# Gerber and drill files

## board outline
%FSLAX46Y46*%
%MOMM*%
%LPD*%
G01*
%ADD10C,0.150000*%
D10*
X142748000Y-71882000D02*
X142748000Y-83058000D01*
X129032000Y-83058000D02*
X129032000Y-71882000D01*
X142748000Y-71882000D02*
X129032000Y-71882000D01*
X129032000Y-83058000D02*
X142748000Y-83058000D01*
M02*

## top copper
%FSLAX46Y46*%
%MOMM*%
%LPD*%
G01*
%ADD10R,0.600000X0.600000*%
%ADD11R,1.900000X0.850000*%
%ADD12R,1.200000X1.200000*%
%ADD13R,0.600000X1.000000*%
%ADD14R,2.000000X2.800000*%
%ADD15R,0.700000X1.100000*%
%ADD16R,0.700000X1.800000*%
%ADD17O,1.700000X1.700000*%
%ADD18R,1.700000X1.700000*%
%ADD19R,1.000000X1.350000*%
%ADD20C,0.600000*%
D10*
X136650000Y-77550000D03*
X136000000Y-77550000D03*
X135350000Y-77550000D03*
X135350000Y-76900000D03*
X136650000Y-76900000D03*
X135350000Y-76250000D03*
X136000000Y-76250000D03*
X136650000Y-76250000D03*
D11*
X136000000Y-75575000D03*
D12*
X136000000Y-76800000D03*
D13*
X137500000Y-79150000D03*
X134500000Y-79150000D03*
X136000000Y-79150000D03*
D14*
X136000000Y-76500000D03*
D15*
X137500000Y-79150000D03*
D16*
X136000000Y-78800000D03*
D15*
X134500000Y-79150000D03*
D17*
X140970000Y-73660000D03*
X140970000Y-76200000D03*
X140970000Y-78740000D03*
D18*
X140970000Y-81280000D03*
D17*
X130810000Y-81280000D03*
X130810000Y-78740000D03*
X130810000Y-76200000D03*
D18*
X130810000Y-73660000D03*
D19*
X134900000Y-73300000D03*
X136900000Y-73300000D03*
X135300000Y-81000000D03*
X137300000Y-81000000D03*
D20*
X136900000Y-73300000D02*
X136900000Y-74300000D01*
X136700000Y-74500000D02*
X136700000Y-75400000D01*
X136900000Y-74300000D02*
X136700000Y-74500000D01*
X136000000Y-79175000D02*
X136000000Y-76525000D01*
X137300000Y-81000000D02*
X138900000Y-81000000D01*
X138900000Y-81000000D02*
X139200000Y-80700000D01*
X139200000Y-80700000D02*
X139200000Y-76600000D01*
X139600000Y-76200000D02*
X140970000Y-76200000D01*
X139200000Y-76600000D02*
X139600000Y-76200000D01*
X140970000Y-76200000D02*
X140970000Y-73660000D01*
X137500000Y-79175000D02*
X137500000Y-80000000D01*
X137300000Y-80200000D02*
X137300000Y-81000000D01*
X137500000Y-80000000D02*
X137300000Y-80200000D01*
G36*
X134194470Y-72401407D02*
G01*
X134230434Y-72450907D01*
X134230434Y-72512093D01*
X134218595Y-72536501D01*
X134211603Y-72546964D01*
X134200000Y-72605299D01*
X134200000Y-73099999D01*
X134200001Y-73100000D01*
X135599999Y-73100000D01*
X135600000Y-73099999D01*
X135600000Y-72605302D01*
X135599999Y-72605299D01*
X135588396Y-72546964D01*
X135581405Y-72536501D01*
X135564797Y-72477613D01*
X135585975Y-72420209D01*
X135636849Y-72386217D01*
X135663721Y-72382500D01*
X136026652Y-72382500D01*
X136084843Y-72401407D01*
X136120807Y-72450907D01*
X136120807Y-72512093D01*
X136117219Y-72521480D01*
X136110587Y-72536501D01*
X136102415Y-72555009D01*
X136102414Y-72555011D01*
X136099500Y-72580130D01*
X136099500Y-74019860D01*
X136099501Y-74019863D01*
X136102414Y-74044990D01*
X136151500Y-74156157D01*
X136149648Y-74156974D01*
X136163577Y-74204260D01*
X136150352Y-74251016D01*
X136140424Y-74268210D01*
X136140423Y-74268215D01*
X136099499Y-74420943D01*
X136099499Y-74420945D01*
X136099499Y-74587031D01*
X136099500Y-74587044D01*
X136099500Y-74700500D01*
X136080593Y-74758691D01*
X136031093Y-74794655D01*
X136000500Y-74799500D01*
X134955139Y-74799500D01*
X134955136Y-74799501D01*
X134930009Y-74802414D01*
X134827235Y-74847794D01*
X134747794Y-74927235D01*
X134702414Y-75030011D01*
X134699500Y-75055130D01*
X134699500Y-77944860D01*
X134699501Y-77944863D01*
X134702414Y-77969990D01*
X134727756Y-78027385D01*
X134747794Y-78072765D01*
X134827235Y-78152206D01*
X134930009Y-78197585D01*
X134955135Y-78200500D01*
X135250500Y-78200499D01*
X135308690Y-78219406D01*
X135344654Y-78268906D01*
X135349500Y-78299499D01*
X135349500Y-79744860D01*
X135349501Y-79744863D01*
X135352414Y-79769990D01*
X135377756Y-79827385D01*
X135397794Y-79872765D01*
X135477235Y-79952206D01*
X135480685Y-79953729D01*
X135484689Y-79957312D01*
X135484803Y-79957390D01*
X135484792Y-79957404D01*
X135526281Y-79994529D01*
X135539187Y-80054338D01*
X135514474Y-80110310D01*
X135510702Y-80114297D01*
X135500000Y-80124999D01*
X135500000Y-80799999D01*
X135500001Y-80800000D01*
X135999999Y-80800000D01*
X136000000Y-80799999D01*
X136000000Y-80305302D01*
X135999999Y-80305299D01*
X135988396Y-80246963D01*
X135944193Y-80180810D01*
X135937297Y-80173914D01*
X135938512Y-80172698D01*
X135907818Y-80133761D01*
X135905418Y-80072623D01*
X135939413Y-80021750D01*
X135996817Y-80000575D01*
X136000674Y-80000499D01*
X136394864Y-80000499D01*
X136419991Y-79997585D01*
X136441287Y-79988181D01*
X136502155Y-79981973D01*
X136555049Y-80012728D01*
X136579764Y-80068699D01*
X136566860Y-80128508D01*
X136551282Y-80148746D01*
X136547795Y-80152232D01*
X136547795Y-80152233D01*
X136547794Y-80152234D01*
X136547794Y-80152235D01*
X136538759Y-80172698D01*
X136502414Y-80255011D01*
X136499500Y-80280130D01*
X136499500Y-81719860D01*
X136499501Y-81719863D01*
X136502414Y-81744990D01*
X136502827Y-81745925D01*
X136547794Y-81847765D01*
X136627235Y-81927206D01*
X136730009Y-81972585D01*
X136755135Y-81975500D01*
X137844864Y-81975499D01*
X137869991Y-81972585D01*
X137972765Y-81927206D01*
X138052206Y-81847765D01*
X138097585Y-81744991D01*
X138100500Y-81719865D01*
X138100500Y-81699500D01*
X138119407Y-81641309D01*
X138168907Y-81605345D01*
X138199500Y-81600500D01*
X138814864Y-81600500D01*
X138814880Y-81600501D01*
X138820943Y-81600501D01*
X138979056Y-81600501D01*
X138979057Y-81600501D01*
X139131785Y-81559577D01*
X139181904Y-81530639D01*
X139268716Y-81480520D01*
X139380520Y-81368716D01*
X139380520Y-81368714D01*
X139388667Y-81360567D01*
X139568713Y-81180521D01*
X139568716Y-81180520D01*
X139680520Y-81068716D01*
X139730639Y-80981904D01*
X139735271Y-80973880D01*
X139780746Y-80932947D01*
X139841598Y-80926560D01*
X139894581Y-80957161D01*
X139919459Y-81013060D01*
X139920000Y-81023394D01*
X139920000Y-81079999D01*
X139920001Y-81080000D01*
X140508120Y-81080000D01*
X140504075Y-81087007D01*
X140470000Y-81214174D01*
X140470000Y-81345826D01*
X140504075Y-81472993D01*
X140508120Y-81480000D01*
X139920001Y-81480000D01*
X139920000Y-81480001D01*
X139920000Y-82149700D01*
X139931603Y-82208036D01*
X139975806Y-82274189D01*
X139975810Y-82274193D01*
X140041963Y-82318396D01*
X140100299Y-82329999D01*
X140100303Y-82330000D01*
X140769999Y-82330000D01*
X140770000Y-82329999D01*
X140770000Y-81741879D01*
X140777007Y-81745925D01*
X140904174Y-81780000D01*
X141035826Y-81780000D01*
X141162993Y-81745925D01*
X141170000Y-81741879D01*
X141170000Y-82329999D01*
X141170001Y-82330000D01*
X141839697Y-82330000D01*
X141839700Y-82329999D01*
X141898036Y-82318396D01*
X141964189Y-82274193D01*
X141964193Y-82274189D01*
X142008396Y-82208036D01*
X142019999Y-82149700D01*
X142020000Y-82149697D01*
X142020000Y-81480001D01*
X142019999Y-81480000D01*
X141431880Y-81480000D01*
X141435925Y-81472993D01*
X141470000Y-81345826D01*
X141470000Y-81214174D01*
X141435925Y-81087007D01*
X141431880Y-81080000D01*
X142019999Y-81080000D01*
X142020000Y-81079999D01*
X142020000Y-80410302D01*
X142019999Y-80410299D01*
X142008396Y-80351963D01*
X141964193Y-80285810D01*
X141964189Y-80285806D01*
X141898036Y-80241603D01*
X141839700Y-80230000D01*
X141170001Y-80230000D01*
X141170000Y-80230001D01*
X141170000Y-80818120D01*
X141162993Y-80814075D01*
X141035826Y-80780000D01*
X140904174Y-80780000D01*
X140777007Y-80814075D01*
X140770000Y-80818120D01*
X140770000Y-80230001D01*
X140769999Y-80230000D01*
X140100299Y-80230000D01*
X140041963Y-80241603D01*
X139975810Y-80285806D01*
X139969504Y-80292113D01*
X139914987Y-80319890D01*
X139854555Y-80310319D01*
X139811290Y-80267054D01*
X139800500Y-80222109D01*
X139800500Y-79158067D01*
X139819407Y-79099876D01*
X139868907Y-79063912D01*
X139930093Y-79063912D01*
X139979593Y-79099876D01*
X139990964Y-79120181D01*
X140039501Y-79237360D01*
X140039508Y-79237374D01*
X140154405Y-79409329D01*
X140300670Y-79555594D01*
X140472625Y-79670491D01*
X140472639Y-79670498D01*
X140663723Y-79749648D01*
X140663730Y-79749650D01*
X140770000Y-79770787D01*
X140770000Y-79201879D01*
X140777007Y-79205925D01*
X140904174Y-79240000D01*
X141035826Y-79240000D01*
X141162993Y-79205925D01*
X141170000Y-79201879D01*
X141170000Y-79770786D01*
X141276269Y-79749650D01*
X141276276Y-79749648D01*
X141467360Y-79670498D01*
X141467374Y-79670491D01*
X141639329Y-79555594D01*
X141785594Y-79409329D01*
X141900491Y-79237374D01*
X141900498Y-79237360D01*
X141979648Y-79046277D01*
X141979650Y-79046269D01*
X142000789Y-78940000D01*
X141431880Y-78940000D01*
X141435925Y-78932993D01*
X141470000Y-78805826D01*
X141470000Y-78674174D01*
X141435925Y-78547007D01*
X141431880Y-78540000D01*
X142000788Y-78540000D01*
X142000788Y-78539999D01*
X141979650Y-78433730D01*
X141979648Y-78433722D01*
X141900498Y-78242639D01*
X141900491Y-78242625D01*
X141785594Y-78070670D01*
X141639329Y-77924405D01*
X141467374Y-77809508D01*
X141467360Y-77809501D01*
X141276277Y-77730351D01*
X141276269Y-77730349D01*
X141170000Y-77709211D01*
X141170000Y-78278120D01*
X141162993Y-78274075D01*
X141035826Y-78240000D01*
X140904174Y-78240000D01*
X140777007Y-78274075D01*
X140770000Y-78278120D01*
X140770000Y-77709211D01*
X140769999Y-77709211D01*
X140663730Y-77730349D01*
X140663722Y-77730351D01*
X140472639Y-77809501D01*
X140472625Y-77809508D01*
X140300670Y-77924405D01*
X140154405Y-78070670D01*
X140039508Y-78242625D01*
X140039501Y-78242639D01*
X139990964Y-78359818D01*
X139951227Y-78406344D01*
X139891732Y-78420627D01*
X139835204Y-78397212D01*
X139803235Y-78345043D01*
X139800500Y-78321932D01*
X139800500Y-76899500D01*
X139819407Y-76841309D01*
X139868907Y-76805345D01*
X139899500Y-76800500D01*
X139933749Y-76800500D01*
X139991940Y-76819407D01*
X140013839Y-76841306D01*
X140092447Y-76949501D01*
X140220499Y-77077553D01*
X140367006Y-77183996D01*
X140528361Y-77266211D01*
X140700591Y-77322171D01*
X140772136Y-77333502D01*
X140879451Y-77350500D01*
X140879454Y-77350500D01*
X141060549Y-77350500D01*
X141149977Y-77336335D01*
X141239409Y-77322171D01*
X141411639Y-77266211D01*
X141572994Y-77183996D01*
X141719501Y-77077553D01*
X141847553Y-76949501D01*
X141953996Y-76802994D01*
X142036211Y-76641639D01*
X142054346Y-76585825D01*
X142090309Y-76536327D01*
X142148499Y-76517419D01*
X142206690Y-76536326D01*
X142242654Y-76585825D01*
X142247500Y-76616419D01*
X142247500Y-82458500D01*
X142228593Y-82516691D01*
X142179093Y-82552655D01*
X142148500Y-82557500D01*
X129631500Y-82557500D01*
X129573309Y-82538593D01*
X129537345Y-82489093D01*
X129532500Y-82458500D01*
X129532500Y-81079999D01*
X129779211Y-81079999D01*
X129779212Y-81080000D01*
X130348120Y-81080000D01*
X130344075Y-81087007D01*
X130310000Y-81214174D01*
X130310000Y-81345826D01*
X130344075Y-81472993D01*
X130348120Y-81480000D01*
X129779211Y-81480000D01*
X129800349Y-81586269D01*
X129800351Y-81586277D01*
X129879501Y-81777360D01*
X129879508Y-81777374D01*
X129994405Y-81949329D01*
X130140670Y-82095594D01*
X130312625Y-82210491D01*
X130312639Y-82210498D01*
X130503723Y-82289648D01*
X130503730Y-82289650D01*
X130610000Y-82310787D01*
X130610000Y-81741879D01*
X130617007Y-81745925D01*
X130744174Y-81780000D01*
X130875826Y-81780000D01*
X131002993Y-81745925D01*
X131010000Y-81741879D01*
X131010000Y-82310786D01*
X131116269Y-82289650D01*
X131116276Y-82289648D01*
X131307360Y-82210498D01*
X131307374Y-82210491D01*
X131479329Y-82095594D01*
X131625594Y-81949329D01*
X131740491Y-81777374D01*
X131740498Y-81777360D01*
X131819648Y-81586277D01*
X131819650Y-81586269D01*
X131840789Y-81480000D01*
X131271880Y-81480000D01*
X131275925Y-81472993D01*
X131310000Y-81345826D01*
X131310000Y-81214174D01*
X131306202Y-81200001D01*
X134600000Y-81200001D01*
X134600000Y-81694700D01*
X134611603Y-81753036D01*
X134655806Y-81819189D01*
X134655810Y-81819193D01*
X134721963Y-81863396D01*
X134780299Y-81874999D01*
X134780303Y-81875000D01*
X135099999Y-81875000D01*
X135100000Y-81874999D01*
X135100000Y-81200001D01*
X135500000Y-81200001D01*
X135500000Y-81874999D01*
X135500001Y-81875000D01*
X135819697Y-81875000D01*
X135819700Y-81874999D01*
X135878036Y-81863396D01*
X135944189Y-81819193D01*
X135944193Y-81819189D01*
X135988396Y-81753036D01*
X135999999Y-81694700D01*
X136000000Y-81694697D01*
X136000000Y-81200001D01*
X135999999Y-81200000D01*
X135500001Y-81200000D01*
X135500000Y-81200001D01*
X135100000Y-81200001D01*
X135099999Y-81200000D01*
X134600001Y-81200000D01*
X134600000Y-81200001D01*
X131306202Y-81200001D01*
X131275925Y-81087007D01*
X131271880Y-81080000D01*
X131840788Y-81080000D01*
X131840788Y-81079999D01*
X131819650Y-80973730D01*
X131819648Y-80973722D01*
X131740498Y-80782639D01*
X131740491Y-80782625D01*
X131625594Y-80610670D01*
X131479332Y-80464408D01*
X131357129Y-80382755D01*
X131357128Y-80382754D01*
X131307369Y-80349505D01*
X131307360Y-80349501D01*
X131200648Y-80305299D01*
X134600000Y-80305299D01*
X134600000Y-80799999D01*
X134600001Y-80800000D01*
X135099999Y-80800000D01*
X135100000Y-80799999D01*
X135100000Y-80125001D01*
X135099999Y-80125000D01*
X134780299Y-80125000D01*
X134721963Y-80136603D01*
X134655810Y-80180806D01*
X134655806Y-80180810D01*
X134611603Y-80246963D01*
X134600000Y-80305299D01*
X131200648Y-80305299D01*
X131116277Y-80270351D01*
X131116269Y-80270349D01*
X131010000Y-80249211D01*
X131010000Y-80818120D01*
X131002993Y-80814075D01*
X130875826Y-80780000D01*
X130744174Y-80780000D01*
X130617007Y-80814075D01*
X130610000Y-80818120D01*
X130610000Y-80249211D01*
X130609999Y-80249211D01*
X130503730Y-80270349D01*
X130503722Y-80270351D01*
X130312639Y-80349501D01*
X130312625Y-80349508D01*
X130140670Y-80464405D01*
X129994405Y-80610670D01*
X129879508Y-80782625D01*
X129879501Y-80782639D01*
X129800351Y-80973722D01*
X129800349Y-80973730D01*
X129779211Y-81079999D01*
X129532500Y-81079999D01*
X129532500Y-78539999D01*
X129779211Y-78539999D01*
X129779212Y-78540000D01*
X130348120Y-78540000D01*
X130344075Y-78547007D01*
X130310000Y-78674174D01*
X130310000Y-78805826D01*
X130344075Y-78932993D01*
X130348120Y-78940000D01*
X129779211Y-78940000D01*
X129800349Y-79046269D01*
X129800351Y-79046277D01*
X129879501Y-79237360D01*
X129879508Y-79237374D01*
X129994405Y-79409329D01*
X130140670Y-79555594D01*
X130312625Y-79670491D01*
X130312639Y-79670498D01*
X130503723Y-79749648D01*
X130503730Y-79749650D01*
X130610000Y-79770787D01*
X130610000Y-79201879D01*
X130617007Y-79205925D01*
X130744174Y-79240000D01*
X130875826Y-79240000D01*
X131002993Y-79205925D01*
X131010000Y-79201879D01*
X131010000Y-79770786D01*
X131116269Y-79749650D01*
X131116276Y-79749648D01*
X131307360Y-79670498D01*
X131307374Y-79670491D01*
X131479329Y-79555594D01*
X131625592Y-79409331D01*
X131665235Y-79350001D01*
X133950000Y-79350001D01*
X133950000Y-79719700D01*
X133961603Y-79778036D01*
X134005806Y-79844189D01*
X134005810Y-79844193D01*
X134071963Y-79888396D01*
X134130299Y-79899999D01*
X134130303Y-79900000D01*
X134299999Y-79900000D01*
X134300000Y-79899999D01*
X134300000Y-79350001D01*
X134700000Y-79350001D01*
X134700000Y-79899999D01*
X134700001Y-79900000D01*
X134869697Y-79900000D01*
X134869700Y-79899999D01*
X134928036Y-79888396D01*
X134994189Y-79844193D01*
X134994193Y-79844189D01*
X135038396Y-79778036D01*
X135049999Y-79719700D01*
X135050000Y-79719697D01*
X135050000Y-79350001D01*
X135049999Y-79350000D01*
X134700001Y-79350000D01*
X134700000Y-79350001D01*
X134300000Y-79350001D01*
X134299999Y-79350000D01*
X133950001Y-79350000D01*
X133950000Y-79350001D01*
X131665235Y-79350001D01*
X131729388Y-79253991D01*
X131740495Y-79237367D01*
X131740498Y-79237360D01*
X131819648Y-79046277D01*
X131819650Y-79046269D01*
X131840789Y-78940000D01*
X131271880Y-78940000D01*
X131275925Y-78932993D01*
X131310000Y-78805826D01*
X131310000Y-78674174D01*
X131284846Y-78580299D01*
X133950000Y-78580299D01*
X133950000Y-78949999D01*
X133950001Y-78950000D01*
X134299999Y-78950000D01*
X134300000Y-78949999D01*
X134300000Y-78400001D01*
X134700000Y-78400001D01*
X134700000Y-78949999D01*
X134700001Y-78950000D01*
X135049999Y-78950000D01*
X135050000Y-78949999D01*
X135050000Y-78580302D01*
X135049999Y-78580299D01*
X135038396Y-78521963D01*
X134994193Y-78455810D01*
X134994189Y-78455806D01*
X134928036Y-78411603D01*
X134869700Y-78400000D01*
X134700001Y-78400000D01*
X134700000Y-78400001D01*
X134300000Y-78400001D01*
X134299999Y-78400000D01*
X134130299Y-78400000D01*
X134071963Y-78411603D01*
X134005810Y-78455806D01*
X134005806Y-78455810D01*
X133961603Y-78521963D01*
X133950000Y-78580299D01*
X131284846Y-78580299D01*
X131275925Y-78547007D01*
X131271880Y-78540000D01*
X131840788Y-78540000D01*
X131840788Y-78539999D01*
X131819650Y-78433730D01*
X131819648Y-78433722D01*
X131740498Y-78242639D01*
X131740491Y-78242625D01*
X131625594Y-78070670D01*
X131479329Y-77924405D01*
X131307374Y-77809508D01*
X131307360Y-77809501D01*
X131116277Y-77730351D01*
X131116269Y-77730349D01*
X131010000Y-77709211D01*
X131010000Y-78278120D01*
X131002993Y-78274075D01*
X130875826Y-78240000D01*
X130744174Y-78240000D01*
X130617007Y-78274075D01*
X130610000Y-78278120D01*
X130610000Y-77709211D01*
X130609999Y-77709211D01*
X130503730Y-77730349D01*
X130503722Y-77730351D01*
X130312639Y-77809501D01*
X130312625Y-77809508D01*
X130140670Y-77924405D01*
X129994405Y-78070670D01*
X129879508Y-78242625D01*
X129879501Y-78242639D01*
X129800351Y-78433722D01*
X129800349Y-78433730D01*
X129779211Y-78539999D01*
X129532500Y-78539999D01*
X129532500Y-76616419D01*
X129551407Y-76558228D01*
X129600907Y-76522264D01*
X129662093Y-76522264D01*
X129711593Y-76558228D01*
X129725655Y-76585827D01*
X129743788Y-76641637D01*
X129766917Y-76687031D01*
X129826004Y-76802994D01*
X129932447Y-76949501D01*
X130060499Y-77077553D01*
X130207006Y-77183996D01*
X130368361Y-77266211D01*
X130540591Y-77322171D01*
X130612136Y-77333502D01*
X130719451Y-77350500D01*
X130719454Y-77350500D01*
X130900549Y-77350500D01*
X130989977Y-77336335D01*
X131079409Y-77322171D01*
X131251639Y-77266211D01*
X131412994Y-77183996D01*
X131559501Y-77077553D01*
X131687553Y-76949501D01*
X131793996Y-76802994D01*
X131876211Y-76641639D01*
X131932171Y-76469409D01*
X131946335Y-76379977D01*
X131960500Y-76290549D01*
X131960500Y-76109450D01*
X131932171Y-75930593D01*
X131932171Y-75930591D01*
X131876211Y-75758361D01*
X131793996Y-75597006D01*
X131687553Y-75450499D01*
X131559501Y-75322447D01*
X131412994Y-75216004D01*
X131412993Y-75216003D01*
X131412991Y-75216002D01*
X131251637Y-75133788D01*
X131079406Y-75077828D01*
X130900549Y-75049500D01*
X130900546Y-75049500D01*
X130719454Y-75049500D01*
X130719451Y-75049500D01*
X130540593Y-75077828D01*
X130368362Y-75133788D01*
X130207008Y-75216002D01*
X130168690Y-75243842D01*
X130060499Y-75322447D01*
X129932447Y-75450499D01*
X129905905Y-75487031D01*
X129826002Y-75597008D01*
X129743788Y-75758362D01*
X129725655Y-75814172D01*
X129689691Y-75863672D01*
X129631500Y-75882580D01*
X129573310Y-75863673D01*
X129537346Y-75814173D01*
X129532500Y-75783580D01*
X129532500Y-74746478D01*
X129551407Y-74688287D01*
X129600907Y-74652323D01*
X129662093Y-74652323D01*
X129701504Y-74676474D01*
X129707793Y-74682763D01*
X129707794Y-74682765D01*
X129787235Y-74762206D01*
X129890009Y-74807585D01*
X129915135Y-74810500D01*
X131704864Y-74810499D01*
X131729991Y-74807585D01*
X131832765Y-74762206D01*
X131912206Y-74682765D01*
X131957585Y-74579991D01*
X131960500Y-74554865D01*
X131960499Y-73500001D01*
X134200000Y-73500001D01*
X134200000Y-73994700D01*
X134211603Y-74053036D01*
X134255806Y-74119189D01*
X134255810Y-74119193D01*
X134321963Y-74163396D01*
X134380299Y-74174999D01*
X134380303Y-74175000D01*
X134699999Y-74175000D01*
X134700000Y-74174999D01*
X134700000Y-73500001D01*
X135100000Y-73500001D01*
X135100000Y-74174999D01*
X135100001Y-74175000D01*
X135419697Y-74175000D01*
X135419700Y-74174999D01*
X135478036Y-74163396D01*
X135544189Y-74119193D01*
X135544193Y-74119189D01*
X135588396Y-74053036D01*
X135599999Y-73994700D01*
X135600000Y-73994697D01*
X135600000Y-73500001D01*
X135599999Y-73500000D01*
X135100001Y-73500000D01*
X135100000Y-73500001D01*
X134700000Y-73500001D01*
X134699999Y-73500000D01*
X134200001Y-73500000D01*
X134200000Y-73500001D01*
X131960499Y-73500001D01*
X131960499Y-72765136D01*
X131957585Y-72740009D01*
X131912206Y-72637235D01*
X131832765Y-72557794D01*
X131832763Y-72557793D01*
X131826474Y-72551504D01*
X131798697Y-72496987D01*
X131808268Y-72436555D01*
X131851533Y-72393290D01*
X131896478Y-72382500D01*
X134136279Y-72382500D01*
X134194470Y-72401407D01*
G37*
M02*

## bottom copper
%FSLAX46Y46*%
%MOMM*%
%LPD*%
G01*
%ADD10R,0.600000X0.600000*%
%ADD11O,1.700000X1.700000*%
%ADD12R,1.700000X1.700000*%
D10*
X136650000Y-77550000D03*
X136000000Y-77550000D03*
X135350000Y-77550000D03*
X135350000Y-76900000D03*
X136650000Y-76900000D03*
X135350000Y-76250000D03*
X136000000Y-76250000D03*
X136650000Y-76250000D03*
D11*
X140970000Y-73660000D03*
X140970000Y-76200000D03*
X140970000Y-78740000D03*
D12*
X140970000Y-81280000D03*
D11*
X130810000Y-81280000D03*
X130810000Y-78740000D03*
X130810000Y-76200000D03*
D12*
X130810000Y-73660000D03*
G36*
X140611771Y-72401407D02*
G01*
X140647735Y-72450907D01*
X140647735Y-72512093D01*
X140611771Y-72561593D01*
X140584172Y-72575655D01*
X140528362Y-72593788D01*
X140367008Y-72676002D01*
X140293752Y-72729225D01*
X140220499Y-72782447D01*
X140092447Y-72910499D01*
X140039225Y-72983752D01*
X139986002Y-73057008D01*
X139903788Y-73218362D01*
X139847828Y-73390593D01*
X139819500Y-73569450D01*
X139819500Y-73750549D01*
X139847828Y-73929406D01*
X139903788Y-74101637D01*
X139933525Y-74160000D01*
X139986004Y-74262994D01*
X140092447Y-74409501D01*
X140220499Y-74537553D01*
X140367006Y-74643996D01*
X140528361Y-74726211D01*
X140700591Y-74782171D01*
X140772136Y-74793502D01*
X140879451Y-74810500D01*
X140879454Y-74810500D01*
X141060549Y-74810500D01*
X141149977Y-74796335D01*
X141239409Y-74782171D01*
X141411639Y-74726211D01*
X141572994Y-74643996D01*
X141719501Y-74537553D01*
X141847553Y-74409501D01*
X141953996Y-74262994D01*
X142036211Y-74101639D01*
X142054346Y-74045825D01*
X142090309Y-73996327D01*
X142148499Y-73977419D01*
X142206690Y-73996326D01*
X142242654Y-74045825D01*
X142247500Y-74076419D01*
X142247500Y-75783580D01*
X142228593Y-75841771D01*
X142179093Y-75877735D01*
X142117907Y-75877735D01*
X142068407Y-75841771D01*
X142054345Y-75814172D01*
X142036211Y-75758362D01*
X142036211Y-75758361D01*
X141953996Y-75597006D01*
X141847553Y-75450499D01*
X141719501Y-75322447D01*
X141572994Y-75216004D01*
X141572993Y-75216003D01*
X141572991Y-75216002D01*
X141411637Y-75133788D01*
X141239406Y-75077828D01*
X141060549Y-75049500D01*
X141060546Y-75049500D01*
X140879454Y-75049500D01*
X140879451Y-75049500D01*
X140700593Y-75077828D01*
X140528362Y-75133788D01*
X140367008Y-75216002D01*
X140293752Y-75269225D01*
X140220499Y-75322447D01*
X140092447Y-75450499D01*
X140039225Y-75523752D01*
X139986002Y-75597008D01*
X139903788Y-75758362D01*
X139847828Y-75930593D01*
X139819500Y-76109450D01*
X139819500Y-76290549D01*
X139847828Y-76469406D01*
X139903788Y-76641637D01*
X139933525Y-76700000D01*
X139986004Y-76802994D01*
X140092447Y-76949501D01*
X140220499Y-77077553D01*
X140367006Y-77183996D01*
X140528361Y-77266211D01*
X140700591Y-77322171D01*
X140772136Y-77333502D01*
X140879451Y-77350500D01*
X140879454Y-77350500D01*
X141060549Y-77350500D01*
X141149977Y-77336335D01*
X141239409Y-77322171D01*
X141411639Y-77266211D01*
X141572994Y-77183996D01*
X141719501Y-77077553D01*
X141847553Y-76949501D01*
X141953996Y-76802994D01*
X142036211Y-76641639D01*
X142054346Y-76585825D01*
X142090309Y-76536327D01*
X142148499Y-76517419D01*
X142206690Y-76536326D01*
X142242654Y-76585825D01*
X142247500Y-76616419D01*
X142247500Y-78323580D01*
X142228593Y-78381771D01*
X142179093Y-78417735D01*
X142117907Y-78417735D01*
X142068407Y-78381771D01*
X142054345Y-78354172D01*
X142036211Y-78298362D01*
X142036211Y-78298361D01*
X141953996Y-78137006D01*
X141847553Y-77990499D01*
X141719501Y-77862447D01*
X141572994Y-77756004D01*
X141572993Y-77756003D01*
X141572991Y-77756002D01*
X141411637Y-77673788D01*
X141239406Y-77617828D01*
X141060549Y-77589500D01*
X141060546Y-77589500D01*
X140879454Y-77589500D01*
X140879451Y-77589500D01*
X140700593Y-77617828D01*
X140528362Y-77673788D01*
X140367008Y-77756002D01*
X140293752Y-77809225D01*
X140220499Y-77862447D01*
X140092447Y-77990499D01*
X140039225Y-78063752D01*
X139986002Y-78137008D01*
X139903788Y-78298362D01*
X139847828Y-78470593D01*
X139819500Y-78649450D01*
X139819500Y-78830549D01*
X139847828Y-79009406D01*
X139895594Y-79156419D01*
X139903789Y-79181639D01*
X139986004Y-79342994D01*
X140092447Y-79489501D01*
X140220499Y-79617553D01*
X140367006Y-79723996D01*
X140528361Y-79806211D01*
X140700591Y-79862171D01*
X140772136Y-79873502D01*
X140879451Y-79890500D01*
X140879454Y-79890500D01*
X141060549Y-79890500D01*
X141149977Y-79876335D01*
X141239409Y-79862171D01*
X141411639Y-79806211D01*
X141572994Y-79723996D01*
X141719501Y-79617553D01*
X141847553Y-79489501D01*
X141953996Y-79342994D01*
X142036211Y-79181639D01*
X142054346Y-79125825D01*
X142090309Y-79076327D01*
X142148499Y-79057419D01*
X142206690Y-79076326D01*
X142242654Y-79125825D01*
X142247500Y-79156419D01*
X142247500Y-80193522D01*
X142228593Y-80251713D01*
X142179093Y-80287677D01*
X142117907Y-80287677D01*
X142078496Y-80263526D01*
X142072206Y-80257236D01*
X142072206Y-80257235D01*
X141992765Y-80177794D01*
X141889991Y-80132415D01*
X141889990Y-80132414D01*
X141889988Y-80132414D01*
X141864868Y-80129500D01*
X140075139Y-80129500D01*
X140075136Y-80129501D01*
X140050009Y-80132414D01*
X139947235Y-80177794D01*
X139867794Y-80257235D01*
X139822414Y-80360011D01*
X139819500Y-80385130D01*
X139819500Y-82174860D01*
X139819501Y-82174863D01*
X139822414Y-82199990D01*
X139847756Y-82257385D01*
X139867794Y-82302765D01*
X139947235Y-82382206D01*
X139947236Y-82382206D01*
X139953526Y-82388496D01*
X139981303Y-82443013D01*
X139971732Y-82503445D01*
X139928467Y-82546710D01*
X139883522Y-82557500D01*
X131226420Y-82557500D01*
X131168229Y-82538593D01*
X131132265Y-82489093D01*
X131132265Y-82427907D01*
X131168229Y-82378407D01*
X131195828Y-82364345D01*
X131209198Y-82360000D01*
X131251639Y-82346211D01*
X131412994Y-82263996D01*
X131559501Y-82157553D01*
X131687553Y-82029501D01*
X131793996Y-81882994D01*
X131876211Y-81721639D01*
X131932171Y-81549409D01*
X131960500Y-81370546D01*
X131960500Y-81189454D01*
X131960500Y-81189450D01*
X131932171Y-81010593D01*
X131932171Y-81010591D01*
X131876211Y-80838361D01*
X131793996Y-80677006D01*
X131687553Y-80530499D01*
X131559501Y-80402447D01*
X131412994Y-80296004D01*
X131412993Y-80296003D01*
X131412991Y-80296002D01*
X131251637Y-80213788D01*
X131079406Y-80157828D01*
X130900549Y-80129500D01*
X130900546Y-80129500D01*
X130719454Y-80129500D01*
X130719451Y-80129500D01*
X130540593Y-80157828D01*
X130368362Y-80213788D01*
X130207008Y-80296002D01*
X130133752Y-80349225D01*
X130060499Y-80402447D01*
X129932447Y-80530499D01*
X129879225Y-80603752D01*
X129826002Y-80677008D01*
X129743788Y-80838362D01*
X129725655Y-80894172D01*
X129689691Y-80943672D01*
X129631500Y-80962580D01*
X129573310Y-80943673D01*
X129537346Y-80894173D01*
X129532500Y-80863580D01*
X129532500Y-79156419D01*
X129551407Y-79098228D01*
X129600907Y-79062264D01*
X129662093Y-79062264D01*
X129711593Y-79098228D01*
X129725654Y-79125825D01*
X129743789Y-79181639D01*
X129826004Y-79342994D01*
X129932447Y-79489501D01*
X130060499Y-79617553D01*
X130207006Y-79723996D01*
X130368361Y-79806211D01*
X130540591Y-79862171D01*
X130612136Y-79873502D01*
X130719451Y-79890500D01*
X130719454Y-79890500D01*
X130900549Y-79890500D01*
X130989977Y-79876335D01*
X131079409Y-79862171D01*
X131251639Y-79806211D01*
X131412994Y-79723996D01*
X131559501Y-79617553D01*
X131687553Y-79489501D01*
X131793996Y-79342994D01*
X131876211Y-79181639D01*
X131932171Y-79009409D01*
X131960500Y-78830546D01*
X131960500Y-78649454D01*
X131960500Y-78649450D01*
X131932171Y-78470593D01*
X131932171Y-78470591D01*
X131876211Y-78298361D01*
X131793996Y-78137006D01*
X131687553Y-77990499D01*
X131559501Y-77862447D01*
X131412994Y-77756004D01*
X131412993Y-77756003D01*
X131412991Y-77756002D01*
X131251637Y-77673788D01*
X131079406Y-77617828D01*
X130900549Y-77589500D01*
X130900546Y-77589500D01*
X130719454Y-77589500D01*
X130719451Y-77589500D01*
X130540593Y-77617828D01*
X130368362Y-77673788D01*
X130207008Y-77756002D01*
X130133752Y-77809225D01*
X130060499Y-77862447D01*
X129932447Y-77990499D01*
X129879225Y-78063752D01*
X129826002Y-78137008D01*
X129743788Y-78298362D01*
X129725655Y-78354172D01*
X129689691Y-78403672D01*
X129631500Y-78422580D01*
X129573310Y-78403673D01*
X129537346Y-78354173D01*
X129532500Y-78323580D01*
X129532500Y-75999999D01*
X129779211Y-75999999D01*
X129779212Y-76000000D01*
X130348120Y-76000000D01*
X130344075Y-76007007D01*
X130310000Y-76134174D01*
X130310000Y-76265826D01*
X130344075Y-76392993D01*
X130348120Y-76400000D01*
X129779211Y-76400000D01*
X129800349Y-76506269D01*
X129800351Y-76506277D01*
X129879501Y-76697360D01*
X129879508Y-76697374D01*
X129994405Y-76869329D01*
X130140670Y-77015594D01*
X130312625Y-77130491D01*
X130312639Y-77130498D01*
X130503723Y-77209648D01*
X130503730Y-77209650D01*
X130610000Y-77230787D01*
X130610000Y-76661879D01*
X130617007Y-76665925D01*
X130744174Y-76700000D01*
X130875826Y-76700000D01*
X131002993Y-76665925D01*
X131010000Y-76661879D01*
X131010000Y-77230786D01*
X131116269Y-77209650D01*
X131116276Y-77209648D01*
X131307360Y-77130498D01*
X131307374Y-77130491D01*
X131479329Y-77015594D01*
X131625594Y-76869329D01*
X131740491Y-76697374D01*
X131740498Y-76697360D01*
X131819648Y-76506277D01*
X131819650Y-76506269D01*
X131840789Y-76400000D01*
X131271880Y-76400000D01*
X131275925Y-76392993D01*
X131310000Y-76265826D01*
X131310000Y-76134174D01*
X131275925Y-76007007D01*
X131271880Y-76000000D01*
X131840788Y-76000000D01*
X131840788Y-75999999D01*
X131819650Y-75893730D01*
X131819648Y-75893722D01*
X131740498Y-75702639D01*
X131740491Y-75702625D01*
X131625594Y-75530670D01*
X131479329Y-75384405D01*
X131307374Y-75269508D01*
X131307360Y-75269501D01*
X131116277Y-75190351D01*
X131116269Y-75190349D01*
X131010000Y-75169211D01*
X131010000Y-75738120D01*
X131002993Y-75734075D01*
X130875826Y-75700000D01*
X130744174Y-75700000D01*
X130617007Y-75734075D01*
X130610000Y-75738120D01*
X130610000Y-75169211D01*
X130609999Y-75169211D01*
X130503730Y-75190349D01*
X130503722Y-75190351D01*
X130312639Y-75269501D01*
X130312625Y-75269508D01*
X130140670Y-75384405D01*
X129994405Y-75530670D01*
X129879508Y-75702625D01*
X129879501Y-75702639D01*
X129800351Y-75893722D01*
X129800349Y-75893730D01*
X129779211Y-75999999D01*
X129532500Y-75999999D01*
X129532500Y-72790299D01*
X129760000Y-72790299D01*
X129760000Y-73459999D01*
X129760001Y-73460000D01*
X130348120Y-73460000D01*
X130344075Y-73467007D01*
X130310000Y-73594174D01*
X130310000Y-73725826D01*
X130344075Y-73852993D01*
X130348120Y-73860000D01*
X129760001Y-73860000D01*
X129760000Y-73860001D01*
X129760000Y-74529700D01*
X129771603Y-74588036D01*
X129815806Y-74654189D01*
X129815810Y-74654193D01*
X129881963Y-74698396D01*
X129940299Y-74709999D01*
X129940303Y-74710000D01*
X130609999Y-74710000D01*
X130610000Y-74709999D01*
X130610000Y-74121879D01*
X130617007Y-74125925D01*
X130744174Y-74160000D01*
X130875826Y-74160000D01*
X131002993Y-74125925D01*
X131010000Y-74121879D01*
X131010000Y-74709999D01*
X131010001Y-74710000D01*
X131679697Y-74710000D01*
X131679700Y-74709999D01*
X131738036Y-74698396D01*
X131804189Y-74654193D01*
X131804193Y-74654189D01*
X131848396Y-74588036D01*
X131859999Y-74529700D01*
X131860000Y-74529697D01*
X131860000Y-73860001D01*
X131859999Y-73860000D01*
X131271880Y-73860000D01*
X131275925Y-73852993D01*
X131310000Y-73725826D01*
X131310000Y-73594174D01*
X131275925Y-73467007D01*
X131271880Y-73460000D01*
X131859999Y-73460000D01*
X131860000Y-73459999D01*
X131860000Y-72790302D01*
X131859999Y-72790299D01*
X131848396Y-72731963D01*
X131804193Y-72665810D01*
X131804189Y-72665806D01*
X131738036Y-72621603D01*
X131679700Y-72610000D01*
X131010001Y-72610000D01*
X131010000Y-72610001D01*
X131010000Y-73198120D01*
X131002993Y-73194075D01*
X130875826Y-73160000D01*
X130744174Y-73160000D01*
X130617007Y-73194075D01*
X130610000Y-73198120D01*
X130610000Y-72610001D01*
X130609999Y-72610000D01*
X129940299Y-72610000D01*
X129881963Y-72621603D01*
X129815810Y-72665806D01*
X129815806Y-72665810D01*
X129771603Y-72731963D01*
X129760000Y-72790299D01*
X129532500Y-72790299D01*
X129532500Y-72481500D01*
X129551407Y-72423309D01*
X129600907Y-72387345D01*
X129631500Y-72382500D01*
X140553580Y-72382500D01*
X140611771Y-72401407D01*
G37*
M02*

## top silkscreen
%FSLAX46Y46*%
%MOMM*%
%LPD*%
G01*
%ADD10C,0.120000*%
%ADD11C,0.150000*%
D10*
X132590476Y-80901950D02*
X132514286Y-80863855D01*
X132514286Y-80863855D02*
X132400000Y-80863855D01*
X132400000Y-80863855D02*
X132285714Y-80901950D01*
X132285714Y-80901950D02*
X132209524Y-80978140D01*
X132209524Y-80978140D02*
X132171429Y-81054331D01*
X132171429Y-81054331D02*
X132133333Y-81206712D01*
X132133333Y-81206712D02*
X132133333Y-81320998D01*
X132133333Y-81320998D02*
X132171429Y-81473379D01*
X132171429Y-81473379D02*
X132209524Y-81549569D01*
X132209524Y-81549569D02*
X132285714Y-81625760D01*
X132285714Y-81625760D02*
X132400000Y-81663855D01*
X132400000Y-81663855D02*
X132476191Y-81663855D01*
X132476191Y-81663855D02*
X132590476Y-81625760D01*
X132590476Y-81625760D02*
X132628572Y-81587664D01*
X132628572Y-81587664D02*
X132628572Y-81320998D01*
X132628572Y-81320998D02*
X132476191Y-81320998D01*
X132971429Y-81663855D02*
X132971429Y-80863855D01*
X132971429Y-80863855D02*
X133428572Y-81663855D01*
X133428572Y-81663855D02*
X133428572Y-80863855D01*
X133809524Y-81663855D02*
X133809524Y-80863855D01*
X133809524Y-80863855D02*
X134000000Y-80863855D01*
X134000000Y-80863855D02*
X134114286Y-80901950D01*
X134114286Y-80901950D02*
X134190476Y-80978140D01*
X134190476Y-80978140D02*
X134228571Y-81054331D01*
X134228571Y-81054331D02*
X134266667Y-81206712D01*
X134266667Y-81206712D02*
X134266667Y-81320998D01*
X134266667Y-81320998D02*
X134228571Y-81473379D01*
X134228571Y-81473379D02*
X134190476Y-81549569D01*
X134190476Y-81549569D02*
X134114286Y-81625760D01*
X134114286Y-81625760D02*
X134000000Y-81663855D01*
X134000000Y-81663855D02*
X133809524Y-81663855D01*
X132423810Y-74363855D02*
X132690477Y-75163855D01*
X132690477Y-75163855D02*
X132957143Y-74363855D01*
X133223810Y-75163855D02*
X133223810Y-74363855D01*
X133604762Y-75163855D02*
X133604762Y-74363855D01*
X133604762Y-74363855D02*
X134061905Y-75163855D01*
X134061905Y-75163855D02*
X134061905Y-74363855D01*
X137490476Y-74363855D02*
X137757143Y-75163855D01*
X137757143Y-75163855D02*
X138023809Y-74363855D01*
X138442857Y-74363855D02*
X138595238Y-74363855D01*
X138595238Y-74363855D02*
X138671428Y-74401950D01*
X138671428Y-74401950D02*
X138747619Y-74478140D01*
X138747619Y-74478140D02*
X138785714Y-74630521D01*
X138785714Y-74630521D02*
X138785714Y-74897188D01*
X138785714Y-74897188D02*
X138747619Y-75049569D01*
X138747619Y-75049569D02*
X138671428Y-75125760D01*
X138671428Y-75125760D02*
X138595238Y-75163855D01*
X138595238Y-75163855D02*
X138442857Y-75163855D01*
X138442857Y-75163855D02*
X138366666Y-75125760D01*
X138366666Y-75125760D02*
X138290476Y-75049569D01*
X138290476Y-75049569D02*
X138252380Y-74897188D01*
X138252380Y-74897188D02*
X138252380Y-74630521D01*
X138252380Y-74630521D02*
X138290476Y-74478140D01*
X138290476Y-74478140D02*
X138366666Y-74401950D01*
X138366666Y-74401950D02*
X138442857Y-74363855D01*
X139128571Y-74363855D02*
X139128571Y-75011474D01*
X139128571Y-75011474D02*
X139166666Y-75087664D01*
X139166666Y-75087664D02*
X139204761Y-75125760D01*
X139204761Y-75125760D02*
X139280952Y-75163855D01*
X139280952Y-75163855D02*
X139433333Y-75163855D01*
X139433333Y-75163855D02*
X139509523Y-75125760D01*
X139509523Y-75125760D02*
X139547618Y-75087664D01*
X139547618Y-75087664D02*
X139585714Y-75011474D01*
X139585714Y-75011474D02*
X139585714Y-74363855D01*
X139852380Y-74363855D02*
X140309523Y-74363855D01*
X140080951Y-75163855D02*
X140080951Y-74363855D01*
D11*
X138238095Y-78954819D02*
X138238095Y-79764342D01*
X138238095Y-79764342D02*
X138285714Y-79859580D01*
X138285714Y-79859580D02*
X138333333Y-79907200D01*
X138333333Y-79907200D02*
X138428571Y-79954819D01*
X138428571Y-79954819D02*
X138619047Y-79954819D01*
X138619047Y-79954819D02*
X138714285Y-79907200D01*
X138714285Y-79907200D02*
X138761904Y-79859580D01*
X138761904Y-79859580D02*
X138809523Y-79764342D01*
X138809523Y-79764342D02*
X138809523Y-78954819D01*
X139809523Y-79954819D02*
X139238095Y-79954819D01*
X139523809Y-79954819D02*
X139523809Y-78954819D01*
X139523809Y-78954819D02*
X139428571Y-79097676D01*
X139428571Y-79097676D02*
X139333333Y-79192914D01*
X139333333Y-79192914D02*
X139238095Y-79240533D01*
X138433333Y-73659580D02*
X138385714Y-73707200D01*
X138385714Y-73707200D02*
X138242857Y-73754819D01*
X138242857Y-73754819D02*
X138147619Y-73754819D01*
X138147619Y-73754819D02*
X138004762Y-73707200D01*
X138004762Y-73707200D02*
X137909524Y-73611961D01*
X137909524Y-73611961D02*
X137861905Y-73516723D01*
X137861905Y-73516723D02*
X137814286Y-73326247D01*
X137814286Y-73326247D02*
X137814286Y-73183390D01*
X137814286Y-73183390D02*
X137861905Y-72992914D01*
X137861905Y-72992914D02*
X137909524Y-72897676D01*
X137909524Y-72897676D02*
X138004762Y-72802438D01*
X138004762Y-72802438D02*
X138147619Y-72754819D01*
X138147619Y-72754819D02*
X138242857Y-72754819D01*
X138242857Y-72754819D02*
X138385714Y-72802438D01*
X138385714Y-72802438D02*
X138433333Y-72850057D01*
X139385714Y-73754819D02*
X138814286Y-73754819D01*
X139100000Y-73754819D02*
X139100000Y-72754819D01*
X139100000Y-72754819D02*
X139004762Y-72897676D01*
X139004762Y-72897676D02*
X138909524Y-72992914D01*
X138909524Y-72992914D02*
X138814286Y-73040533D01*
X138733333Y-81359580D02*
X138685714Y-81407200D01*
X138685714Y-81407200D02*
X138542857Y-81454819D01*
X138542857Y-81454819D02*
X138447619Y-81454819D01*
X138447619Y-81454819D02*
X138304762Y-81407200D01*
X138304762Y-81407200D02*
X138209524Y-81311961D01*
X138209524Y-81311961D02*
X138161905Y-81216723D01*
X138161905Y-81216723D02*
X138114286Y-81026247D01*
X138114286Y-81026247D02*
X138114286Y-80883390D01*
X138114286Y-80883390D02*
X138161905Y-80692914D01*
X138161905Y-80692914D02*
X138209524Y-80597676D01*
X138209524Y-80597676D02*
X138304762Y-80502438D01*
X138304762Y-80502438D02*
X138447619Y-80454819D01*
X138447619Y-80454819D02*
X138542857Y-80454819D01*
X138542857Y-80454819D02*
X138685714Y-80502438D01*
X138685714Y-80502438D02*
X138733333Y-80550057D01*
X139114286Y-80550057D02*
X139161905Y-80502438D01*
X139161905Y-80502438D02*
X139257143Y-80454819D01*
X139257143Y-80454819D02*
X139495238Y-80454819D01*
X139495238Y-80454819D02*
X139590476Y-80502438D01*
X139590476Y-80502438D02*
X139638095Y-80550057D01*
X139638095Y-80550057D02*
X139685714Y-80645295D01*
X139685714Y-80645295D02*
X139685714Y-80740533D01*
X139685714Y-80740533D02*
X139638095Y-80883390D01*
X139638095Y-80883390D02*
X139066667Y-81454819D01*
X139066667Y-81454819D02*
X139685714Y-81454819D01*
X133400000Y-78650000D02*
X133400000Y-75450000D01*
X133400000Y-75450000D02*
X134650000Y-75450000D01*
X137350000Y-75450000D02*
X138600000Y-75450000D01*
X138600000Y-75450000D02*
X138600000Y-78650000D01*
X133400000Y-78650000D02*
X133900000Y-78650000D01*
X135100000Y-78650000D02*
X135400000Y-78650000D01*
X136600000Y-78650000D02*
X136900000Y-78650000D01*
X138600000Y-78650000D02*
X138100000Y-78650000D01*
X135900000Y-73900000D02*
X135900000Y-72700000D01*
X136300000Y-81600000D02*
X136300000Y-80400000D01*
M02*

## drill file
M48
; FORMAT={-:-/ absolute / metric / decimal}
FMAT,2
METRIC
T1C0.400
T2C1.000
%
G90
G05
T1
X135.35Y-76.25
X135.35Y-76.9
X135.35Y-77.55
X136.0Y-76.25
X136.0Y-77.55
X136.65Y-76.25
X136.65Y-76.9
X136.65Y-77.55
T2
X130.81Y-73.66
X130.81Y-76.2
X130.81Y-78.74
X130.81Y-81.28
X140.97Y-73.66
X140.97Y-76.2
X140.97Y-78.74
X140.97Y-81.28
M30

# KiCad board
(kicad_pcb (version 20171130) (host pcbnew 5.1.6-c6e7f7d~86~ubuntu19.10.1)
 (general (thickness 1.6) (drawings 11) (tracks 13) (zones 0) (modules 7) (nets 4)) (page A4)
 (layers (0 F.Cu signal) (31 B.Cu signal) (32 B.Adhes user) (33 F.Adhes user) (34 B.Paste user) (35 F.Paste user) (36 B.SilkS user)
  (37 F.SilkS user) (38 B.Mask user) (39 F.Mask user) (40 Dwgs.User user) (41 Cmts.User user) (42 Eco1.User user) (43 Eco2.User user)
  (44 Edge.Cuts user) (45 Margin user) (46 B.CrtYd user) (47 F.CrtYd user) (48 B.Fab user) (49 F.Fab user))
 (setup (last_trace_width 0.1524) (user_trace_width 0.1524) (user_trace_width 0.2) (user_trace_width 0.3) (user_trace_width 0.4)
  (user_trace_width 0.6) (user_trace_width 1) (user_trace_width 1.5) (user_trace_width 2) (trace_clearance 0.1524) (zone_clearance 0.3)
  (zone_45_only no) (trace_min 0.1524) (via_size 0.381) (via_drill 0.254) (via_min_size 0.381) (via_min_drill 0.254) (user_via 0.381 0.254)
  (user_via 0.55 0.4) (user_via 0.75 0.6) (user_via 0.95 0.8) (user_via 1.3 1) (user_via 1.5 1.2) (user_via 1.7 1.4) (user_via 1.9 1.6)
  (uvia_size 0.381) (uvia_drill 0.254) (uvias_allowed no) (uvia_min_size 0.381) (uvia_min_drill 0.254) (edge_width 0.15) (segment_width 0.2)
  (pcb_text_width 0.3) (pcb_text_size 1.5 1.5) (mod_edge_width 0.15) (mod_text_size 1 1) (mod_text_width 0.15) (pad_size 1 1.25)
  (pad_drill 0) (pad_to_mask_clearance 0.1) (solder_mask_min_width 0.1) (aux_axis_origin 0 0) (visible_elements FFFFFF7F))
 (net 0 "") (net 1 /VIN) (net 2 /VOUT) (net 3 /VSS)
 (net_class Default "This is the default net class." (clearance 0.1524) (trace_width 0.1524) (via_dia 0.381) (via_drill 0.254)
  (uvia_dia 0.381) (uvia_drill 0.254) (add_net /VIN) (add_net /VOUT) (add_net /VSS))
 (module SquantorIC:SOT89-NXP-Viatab (layer F.Cu) (at 136 77.4)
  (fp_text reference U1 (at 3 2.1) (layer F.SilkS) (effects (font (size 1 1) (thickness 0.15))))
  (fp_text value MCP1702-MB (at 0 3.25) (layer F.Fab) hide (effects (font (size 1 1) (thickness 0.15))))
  (fp_line (start -2.6 1.25) (end -2.6 -1.95) (layer F.SilkS) (width 0.15))
  (fp_line (start -2.6 -1.95) (end -1.35 -1.95) (layer F.SilkS) (width 0.15))
  (fp_line (start 1.35 -1.95) (end 2.6 -1.95) (layer F.SilkS) (width 0.15))
  (fp_line (start 2.6 -1.95) (end 2.6 1.25) (layer F.SilkS) (width 0.15))
  (fp_line (start -2.6 1.25) (end -2.1 1.25) (layer F.SilkS) (width 0.15))
  (fp_line (start -0.9 1.25) (end -0.6 1.25) (layer F.SilkS) (width 0.15))
  (fp_line (start 0.6 1.25) (end 0.9 1.25) (layer F.SilkS) (width 0.15))
  (fp_line (start 2.6 1.25) (end 2.1 1.25) (layer F.SilkS) (width 0.15))
  (pad 2 thru_hole rect (at 0.65 0.15) (size 0.6 0.6) (drill 0.4) (layers *.Cu *.Mask) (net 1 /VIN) (zone_connect 2))
  (pad 2 thru_hole rect (at 0 0.15) (size 0.6 0.6) (drill 0.4) (layers *.Cu *.Mask) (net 1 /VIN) (zone_connect 2))
  (pad 2 thru_hole rect (at -0.65 0.15) (size 0.6 0.6) (drill 0.4) (layers *.Cu *.Mask) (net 1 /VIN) (zone_connect 2))
  (pad 2 thru_hole rect (at -0.65 -0.5) (size 0.6 0.6) (drill 0.4) (layers *.Cu *.Mask) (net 1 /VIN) (zone_connect 2))
  (pad 2 thru_hole rect (at 0.65 -0.5) (size 0.6 0.6) (drill 0.4) (layers *.Cu *.Mask) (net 1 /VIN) (zone_connect 2))
  (pad 2 thru_hole rect (at -0.65 -1.15 90) (size 0.6 0.6) (drill 0.4) (layers *.Cu *.Mask) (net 1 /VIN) (zone_connect 2))
  (pad 2 thru_hole rect (at 0 -1.15) (size 0.6 0.6) (drill 0.4) (layers *.Cu *.Mask) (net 1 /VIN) (zone_connect 2))
  (pad 2 thru_hole rect (at 0.65 -1.15) (size 0.6 0.6) (drill 0.4) (layers *.Cu *.Mask) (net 1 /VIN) (zone_connect 2))
  (pad 2 smd rect (at 0 -1.825) (size 1.9 0.85) (layers F.Cu F.Paste) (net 1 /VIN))
  (pad 2 smd rect (at 0 -0.6) (size 1.2 1.2) (layers F.Cu F.Paste) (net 1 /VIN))
  (pad 3 smd rect (at 1.5 1.75) (size 0.6 1) (layers F.Cu F.Paste) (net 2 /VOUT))
  (pad 1 smd rect (at -1.5 1.75) (size 0.6 1) (layers F.Cu F.Paste) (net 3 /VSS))
  (pad 2 smd rect (at 0 1.75) (size 0.6 1) (layers F.Cu F.Paste) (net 1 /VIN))
  (pad 2 smd rect (at 0 -0.9) (size 2 2.8) (layers F.Cu F.Mask) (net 1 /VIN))
  (pad 3 smd rect (at 1.5 1.75) (size 0.7 1.1) (layers F.Cu F.Mask) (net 2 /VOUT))
  (pad 2 smd rect (at 0 1.4) (size 0.7 1.8) (layers F.Cu F.Mask) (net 1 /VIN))
  (pad 1 smd rect (at -1.5 1.75) (size 0.7 1.1) (layers F.Cu F.Mask) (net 3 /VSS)))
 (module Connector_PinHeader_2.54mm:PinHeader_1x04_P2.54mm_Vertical (layer B.Cu) (at 140.97 81.28)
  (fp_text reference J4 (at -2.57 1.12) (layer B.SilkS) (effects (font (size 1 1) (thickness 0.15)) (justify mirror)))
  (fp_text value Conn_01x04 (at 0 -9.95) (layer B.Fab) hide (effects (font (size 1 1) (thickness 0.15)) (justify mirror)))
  (pad 4 thru_hole oval (at 0 -7.62) (size 1.7 1.7) (drill 1) (layers *.Cu *.Mask) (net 2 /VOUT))
  (pad 3 thru_hole oval (at 0 -5.08) (size 1.7 1.7) (drill 1) (layers *.Cu *.Mask) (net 2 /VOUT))
  (pad 2 thru_hole oval (at 0 -2.54) (size 1.7 1.7) (drill 1) (layers *.Cu *.Mask) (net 3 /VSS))
  (pad 1 thru_hole rect (at 0 0) (size 1.7 1.7) (drill 1) (layers *.Cu *.Mask) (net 3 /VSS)))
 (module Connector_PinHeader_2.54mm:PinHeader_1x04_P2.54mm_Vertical (layer B.Cu) (at 130.81 73.66 180)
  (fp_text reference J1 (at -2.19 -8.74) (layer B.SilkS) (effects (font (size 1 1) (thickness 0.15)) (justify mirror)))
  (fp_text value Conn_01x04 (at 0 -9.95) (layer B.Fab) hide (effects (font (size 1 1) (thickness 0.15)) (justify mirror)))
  (pad 4 thru_hole oval (at 0 -7.62 180) (size 1.7 1.7) (drill 1) (layers *.Cu *.Mask) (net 3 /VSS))
  (pad 3 thru_hole oval (at 0 -5.08 180) (size 1.7 1.7) (drill 1) (layers *.Cu *.Mask) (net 3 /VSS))
  (pad 2 thru_hole oval (at 0 -2.54 180) (size 1.7 1.7) (drill 1) (layers *.Cu *.Mask) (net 1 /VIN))
  (pad 1 thru_hole rect (at 0 0 180) (size 1.7 1.7) (drill 1) (layers *.Cu *.Mask) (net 1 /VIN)))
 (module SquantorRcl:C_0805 (layer F.Cu) (at 135.9 73.3 180)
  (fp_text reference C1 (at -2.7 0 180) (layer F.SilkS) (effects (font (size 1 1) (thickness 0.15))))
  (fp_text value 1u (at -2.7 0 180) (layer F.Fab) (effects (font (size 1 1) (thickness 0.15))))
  (fp_line (start 0 -0.6) (end 0 0.6) (layer F.SilkS) (width 0.15))
  (pad 2 smd rect (at 1 0 180) (size 1 1.35) (layers F.Cu F.Paste F.Mask) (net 3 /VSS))
  (pad 1 smd rect (at -1 0 180) (size 1 1.35) (layers F.Cu F.Paste F.Mask) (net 1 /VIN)))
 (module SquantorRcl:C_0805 (layer F.Cu) (at 136.3 81 180)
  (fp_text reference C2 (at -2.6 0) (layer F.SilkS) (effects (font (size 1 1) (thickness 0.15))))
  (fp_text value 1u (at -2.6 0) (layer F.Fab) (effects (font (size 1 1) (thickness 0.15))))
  (fp_line (start 0 -0.6) (end 0 0.6) (layer F.SilkS) (width 0.15))
  (pad 2 smd rect (at 1 0 180) (size 1 1.35) (layers F.Cu F.Paste F.Mask) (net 3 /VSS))
  (pad 1 smd rect (at -1 0 180) (size 1 1.35) (layers F.Cu F.Paste F.Mask) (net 2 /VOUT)))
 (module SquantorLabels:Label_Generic (layer B.Cu) (at 136.5 80.1 180)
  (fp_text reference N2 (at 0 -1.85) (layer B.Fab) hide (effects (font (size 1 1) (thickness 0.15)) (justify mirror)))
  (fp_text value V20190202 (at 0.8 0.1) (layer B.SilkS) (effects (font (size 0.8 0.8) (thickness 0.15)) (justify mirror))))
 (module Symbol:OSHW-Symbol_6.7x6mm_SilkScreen (layer B.Cu) (at 135.9 76.3 180)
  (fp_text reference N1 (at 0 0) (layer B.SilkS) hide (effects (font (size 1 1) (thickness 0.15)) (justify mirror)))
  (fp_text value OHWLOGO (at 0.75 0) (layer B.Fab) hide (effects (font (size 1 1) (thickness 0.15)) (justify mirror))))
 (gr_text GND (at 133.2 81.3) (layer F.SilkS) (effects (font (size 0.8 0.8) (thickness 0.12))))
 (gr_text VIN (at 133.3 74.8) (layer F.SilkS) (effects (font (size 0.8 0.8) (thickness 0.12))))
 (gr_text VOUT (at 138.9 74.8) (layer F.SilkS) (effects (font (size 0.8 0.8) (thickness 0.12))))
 (gr_line (start 142.748 71.882) (end 142.748 83.058) (layer Edge.Cuts) (width 0.15))
 (gr_line (start 129.032 83.058) (end 129.032 71.882) (layer Edge.Cuts) (width 0.15))
 (gr_line (start 142.748 71.882) (end 129.032 71.882) (layer Edge.Cuts) (width 0.15))
 (gr_line (start 129.032 83.058) (end 142.748 83.058) (layer Edge.Cuts) (width 0.15))
 (segment (start 136.9 73.3) (end 136.9 74.3) (width 0.6) (layer F.Cu) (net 1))
 (segment (start 136.7 74.5) (end 136.7 75.4) (width 0.6) (layer F.Cu) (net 1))
 (segment (start 136.9 74.3) (end 136.7 74.5) (width 0.6) (layer F.Cu) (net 1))
 (segment (start 136 79.175) (end 136 76.525) (width 0.6) (layer F.Cu) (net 1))
 (segment (start 137.3 81) (end 138.9 81) (width 0.6) (layer F.Cu) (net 2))
 (segment (start 138.9 81) (end 139.2 80.7) (width 0.6) (layer F.Cu) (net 2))
 (segment (start 139.2 80.7) (end 139.2 76.6) (width 0.6) (layer F.Cu) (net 2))
 (segment (start 139.6 76.2) (end 140.97 76.2) (width 0.6) (layer F.Cu) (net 2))
 (segment (start 139.2 76.6) (end 139.6 76.2) (width 0.6) (layer F.Cu) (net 2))
 (segment (start 140.97 76.2) (end 140.97 73.66) (width 0.6) (layer F.Cu) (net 2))
 (segment (start 137.5 79.175) (end 137.5 80) (width 0.6) (layer F.Cu) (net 2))
 (segment (start 137.3 80.2) (end 137.3 81) (width 0.6) (layer F.Cu) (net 2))
 (segment (start 137.5 80) (end 137.3 80.2) (width 0.6) (layer F.Cu) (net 2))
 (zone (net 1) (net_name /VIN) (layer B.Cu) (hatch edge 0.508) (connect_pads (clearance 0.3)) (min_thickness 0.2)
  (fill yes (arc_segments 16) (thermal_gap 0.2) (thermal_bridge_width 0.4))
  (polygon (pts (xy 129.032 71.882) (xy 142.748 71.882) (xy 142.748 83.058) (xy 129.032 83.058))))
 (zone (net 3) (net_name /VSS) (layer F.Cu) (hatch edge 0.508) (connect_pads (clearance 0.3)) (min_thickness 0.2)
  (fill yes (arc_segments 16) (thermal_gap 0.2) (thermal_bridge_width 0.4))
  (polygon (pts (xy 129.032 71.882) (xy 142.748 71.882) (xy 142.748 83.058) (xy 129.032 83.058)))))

